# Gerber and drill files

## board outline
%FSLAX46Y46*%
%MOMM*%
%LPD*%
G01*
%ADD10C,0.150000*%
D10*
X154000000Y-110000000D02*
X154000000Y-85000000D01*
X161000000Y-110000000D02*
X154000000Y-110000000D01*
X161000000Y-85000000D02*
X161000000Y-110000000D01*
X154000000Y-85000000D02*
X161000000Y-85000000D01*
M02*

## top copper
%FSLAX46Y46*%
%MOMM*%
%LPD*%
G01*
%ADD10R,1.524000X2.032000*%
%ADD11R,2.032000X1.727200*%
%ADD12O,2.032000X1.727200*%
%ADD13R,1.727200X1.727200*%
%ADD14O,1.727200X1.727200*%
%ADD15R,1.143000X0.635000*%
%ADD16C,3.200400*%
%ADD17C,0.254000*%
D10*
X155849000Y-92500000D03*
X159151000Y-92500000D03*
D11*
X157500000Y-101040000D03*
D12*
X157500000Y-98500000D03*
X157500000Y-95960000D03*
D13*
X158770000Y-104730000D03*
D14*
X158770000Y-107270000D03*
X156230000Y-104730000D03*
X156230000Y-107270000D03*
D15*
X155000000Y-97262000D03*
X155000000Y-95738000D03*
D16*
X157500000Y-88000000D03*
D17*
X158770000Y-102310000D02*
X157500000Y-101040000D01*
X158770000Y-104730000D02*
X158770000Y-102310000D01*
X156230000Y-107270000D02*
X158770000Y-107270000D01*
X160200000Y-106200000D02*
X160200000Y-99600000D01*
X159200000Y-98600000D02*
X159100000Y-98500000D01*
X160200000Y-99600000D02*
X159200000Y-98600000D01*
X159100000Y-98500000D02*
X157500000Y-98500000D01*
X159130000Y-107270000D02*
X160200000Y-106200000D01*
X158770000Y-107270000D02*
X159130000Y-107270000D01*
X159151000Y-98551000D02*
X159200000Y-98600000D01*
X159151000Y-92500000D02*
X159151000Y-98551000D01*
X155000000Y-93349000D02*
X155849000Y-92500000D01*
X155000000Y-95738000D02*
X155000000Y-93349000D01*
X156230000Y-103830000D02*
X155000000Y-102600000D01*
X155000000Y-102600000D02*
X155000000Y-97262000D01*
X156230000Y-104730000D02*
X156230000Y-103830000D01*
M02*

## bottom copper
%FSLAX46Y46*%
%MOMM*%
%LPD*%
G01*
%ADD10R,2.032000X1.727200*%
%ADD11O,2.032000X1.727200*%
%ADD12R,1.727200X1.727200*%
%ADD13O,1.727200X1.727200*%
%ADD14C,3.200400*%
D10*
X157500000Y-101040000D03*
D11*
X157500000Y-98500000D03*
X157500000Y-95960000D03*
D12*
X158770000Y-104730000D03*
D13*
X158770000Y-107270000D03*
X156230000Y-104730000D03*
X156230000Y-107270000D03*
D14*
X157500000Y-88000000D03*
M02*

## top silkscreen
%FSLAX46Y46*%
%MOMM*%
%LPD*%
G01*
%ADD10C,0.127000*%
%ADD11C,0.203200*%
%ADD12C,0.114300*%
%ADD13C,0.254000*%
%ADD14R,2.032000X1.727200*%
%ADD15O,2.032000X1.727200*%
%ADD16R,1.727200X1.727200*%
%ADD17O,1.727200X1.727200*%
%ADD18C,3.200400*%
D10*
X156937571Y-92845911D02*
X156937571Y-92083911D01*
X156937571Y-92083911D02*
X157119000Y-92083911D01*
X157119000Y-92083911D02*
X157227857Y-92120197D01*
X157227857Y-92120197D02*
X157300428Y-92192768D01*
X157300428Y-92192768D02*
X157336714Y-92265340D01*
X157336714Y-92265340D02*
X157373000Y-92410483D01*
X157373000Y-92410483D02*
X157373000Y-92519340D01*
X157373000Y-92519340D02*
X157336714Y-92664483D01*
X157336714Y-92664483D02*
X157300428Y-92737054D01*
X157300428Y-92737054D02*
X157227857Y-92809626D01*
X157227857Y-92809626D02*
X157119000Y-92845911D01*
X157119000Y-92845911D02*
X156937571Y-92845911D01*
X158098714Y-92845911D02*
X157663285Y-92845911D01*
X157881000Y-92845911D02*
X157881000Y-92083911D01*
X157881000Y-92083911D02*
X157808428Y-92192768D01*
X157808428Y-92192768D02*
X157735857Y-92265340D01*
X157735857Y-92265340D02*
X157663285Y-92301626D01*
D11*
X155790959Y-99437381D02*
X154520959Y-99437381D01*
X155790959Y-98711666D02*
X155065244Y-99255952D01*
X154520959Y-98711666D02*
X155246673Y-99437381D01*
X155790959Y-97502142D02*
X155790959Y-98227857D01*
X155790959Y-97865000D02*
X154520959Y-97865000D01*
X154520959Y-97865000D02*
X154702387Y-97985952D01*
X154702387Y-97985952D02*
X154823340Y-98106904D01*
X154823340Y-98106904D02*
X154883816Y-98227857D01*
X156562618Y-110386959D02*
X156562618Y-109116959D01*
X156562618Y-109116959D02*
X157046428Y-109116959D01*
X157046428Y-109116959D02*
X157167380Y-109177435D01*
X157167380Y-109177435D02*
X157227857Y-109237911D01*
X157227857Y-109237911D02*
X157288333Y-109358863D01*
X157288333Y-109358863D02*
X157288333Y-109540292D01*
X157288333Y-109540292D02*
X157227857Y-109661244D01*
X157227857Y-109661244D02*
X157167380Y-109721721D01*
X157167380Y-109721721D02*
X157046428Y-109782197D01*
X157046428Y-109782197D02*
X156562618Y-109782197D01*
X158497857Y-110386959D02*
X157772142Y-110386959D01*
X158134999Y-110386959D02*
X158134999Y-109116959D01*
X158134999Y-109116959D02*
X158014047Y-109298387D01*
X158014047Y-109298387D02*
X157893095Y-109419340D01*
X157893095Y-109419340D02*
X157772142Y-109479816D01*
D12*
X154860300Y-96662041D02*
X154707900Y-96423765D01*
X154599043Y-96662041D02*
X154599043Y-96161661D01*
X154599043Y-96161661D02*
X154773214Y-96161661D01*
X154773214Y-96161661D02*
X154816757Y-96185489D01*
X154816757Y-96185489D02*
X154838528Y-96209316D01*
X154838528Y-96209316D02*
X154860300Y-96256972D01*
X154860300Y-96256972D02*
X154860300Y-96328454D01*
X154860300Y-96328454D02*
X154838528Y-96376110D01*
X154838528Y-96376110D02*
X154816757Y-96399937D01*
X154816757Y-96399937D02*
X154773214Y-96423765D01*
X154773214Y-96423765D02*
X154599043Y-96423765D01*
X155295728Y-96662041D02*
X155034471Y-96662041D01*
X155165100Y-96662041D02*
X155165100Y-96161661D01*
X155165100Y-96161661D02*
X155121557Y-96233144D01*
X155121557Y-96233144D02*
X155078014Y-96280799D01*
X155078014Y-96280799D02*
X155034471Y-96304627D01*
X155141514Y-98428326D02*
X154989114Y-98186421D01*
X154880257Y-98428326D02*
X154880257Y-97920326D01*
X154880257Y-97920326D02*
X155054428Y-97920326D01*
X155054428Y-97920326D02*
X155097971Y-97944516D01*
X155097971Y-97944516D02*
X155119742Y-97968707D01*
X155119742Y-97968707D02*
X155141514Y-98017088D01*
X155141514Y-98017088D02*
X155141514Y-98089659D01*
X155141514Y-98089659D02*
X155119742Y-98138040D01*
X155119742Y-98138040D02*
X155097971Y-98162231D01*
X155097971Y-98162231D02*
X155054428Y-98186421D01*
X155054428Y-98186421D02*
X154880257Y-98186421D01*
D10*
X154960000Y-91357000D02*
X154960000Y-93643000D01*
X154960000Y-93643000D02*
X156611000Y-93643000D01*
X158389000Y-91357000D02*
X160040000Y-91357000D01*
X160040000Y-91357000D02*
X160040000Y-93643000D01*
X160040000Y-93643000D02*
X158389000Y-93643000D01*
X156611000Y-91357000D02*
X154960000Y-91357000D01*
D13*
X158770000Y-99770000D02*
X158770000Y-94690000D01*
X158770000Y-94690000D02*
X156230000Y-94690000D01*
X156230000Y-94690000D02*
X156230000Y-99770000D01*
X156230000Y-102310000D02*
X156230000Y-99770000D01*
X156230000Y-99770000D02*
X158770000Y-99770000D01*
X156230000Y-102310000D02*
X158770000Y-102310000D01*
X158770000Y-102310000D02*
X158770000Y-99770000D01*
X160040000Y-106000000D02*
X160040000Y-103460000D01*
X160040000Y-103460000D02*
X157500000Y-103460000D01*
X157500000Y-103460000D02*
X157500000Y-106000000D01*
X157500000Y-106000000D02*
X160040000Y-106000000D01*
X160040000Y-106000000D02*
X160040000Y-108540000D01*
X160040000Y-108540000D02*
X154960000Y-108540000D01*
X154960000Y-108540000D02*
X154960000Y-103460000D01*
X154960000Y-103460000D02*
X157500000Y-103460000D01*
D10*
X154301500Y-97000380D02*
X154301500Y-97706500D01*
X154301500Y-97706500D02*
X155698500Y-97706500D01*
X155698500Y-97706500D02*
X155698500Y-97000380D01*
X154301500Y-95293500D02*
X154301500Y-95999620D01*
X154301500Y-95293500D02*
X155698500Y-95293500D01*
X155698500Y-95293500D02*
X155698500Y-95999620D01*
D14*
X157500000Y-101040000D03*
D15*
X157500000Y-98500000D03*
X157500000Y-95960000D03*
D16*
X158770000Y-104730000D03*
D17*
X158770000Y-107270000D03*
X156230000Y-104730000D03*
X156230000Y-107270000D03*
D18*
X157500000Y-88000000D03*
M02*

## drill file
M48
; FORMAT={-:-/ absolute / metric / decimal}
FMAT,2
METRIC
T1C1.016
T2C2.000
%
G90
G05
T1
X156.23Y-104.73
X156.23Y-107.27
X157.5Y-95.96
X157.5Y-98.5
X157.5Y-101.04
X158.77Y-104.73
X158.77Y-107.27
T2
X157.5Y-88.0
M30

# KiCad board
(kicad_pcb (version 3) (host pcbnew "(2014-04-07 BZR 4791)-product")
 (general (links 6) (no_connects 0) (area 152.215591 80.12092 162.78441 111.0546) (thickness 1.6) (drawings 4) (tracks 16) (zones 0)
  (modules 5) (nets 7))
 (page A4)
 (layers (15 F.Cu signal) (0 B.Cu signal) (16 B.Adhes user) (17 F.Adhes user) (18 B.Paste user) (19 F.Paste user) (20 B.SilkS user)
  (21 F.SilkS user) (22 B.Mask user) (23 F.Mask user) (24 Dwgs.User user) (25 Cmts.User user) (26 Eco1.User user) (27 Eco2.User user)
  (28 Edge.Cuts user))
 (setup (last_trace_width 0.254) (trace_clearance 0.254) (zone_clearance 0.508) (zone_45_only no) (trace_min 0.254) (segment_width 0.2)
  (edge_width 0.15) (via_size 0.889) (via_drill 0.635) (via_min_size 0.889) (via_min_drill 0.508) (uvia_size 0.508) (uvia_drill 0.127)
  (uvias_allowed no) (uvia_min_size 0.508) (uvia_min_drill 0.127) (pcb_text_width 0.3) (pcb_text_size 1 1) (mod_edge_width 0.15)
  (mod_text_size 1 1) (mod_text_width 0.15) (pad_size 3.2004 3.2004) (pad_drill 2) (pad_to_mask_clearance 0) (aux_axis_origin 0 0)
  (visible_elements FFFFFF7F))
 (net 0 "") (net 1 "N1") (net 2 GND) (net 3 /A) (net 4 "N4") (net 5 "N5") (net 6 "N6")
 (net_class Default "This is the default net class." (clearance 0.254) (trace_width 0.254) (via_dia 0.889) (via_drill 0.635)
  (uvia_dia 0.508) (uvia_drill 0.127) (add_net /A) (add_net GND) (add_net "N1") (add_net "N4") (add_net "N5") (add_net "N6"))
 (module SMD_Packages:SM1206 (layer F.Cu) (at 157.5 92.5)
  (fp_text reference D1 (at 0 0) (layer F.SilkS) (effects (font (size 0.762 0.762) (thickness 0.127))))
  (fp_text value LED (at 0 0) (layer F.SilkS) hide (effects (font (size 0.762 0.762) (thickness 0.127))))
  (fp_line (start -2.54 -1.143) (end -2.54 1.143) (layer F.SilkS) (width 0.127))
  (fp_line (start -2.54 1.143) (end -0.889 1.143) (layer F.SilkS) (width 0.127))
  (fp_line (start 0.889 -1.143) (end 2.54 -1.143) (layer F.SilkS) (width 0.127))
  (fp_line (start 2.54 -1.143) (end 2.54 1.143) (layer F.SilkS) (width 0.127))
  (fp_line (start 2.54 1.143) (end 0.889 1.143) (layer F.SilkS) (width 0.127))
  (fp_line (start -0.889 -1.143) (end -2.54 -1.143) (layer F.SilkS) (width 0.127))
  (pad 1 smd rect (at -1.651 0) (size 1.524 2.032) (layers F.Cu F.Paste F.Mask) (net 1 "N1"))
  (pad 2 smd rect (at 1.651 0) (size 1.524 2.032) (layers F.Cu F.Paste F.Mask) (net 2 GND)))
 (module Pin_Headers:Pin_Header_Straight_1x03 (layer F.Cu) (at 157.5 98.5 90)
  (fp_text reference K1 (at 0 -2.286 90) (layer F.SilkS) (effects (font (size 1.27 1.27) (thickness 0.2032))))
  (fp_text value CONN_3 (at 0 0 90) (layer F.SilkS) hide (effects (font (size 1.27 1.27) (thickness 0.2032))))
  (fp_line (start -1.27 1.27) (end 3.81 1.27) (layer F.SilkS) (width 0.254))
  (fp_line (start 3.81 1.27) (end 3.81 -1.27) (layer F.SilkS) (width 0.254))
  (fp_line (start 3.81 -1.27) (end -1.27 -1.27) (layer F.SilkS) (width 0.254))
  (fp_line (start -3.81 -1.27) (end -1.27 -1.27) (layer F.SilkS) (width 0.254))
  (fp_line (start -1.27 -1.27) (end -1.27 1.27) (layer F.SilkS) (width 0.254))
  (fp_line (start -3.81 -1.27) (end -3.81 1.27) (layer F.SilkS) (width 0.254))
  (fp_line (start -3.81 1.27) (end -1.27 1.27) (layer F.SilkS) (width 0.254))
  (pad 1 thru_hole rect (at -2.54 0 90) (size 1.7272 2.032) (drill 1.016) (layers *.Cu *.Mask F.SilkS) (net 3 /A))
  (pad 2 thru_hole oval (at 0 0 90) (size 1.7272 2.032) (drill 1.016) (layers *.Cu *.Mask F.SilkS) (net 2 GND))
  (pad 3 thru_hole oval (at 2.54 0 90) (size 1.7272 2.032) (drill 1.016) (layers *.Cu *.Mask F.SilkS) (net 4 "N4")))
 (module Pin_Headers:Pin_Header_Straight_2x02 (layer F.Cu) (at 157.5 106 180)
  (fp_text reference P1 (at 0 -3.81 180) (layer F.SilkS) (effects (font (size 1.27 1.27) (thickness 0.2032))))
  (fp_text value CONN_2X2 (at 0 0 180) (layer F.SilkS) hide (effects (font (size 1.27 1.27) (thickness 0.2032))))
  (fp_line (start -2.54 0) (end -2.54 2.54) (layer F.SilkS) (width 0.254))
  (fp_line (start -2.54 2.54) (end 0 2.54) (layer F.SilkS) (width 0.254))
  (fp_line (start 0 2.54) (end 0 0) (layer F.SilkS) (width 0.254))
  (fp_line (start 0 0) (end -2.54 0) (layer F.SilkS) (width 0.254))
  (fp_line (start -2.54 0) (end -2.54 -2.54) (layer F.SilkS) (width 0.254))
  (fp_line (start -2.54 -2.54) (end 2.54 -2.54) (layer F.SilkS) (width 0.254))
  (fp_line (start 2.54 -2.54) (end 2.54 2.54) (layer F.SilkS) (width 0.254))
  (fp_line (start 2.54 2.54) (end 0 2.54) (layer F.SilkS) (width 0.254))
  (pad 1 thru_hole rect (at -1.27 1.27 180) (size 1.7272 1.7272) (drill 1.016) (layers *.Cu *.Mask F.SilkS) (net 3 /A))
  (pad 2 thru_hole oval (at -1.27 -1.27 180) (size 1.7272 1.7272) (drill 1.016) (layers *.Cu *.Mask F.SilkS) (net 2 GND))
  (pad 3 thru_hole oval (at 1.27 1.27 180) (size 1.7272 1.7272) (drill 1.016) (layers *.Cu *.Mask F.SilkS) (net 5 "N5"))
  (pad 4 thru_hole oval (at 1.27 -1.27 180) (size 1.7272 1.7272) (drill 1.016) (layers *.Cu *.Mask F.SilkS) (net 2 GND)))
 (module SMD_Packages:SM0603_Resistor (layer F.Cu) (at 155 96.5 90)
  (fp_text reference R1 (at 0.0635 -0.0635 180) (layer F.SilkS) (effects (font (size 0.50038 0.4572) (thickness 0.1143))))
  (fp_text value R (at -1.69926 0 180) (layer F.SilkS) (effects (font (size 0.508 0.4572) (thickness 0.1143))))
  (fp_line (start -0.50038 -0.6985) (end -1.2065 -0.6985) (layer F.SilkS) (width 0.127))
  (fp_line (start -1.2065 -0.6985) (end -1.2065 0.6985) (layer F.SilkS) (width 0.127))
  (fp_line (start -1.2065 0.6985) (end -0.50038 0.6985) (layer F.SilkS) (width 0.127))
  (fp_line (start 1.2065 -0.6985) (end 0.50038 -0.6985) (layer F.SilkS) (width 0.127))
  (fp_line (start 1.2065 -0.6985) (end 1.2065 0.6985) (layer F.SilkS) (width 0.127))
  (fp_line (start 1.2065 0.6985) (end 0.50038 0.6985) (layer F.SilkS) (width 0.127))
  (pad 1 smd rect (at -0.762 0 90) (size 0.635 1.143) (layers F.Cu F.Paste F.Mask) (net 5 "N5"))
  (pad 2 smd rect (at 0.762 0 90) (size 0.635 1.143) (layers F.Cu F.Paste F.Mask) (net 1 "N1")))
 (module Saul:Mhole (layer F.Cu) (at 157.5 88)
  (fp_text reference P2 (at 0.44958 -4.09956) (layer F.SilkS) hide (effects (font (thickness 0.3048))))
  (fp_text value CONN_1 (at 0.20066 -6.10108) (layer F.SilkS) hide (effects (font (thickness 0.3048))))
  (pad 1 thru_hole circle (at 0 0) (size 3.2004 3.2004) (drill 2) (layers *.Cu *.Mask F.SilkS) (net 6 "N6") (clearance 1.00076)))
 (gr_line (start 154 110) (end 154 85) (angle 90) (layer Edge.Cuts) (width 0.15))
 (gr_line (start 161 110) (end 154 110) (angle 90) (layer Edge.Cuts) (width 0.15))
 (gr_line (start 161 85) (end 161 110) (angle 90) (layer Edge.Cuts) (width 0.15))
 (gr_line (start 154 85) (end 161 85) (angle 90) (layer Edge.Cuts) (width 0.15))
 (segment (start 158.77 102.31) (end 157.5 101.04) (width 0.254) (layer F.Cu) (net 3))
 (segment (start 158.77 104.73) (end 158.77 102.31) (width 0.254) (layer F.Cu) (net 3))
 (segment (start 156.23 107.27) (end 158.77 107.27) (width 0.254) (layer F.Cu) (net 2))
 (segment (start 160.2 106.2) (end 160.2 99.6) (width 0.254) (layer F.Cu) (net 2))
 (segment (start 159.2 98.6) (end 159.1 98.5) (width 0.254) (layer F.Cu) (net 2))
 (segment (start 160.2 99.6) (end 159.2 98.6) (width 0.254) (layer F.Cu) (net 2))
 (segment (start 159.1 98.5) (end 157.5 98.5) (width 0.254) (layer F.Cu) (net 2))
 (segment (start 159.13 107.27) (end 160.2 106.2) (width 0.254) (layer F.Cu) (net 2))
 (segment (start 158.77 107.27) (end 159.13 107.27) (width 0.254) (layer F.Cu) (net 2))
 (segment (start 159.151 98.551) (end 159.2 98.6) (width 0.254) (layer F.Cu) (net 2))
 (segment (start 159.151 92.5) (end 159.151 98.551) (width 0.254) (layer F.Cu) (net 2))
 (segment (start 155 93.349) (end 155.849 92.5) (width 0.254) (layer F.Cu) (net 1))
 (segment (start 155 95.738) (end 155 93.349) (width 0.254) (layer F.Cu) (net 1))
 (segment (start 156.23 103.83) (end 155 102.6) (width 0.254) (layer F.Cu) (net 5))
 (segment (start 155 102.6) (end 155 97.262) (width 0.254) (layer F.Cu) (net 5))
 (segment (start 156.23 104.73) (end 156.23 103.83) (width 0.254) (layer F.Cu) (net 5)))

